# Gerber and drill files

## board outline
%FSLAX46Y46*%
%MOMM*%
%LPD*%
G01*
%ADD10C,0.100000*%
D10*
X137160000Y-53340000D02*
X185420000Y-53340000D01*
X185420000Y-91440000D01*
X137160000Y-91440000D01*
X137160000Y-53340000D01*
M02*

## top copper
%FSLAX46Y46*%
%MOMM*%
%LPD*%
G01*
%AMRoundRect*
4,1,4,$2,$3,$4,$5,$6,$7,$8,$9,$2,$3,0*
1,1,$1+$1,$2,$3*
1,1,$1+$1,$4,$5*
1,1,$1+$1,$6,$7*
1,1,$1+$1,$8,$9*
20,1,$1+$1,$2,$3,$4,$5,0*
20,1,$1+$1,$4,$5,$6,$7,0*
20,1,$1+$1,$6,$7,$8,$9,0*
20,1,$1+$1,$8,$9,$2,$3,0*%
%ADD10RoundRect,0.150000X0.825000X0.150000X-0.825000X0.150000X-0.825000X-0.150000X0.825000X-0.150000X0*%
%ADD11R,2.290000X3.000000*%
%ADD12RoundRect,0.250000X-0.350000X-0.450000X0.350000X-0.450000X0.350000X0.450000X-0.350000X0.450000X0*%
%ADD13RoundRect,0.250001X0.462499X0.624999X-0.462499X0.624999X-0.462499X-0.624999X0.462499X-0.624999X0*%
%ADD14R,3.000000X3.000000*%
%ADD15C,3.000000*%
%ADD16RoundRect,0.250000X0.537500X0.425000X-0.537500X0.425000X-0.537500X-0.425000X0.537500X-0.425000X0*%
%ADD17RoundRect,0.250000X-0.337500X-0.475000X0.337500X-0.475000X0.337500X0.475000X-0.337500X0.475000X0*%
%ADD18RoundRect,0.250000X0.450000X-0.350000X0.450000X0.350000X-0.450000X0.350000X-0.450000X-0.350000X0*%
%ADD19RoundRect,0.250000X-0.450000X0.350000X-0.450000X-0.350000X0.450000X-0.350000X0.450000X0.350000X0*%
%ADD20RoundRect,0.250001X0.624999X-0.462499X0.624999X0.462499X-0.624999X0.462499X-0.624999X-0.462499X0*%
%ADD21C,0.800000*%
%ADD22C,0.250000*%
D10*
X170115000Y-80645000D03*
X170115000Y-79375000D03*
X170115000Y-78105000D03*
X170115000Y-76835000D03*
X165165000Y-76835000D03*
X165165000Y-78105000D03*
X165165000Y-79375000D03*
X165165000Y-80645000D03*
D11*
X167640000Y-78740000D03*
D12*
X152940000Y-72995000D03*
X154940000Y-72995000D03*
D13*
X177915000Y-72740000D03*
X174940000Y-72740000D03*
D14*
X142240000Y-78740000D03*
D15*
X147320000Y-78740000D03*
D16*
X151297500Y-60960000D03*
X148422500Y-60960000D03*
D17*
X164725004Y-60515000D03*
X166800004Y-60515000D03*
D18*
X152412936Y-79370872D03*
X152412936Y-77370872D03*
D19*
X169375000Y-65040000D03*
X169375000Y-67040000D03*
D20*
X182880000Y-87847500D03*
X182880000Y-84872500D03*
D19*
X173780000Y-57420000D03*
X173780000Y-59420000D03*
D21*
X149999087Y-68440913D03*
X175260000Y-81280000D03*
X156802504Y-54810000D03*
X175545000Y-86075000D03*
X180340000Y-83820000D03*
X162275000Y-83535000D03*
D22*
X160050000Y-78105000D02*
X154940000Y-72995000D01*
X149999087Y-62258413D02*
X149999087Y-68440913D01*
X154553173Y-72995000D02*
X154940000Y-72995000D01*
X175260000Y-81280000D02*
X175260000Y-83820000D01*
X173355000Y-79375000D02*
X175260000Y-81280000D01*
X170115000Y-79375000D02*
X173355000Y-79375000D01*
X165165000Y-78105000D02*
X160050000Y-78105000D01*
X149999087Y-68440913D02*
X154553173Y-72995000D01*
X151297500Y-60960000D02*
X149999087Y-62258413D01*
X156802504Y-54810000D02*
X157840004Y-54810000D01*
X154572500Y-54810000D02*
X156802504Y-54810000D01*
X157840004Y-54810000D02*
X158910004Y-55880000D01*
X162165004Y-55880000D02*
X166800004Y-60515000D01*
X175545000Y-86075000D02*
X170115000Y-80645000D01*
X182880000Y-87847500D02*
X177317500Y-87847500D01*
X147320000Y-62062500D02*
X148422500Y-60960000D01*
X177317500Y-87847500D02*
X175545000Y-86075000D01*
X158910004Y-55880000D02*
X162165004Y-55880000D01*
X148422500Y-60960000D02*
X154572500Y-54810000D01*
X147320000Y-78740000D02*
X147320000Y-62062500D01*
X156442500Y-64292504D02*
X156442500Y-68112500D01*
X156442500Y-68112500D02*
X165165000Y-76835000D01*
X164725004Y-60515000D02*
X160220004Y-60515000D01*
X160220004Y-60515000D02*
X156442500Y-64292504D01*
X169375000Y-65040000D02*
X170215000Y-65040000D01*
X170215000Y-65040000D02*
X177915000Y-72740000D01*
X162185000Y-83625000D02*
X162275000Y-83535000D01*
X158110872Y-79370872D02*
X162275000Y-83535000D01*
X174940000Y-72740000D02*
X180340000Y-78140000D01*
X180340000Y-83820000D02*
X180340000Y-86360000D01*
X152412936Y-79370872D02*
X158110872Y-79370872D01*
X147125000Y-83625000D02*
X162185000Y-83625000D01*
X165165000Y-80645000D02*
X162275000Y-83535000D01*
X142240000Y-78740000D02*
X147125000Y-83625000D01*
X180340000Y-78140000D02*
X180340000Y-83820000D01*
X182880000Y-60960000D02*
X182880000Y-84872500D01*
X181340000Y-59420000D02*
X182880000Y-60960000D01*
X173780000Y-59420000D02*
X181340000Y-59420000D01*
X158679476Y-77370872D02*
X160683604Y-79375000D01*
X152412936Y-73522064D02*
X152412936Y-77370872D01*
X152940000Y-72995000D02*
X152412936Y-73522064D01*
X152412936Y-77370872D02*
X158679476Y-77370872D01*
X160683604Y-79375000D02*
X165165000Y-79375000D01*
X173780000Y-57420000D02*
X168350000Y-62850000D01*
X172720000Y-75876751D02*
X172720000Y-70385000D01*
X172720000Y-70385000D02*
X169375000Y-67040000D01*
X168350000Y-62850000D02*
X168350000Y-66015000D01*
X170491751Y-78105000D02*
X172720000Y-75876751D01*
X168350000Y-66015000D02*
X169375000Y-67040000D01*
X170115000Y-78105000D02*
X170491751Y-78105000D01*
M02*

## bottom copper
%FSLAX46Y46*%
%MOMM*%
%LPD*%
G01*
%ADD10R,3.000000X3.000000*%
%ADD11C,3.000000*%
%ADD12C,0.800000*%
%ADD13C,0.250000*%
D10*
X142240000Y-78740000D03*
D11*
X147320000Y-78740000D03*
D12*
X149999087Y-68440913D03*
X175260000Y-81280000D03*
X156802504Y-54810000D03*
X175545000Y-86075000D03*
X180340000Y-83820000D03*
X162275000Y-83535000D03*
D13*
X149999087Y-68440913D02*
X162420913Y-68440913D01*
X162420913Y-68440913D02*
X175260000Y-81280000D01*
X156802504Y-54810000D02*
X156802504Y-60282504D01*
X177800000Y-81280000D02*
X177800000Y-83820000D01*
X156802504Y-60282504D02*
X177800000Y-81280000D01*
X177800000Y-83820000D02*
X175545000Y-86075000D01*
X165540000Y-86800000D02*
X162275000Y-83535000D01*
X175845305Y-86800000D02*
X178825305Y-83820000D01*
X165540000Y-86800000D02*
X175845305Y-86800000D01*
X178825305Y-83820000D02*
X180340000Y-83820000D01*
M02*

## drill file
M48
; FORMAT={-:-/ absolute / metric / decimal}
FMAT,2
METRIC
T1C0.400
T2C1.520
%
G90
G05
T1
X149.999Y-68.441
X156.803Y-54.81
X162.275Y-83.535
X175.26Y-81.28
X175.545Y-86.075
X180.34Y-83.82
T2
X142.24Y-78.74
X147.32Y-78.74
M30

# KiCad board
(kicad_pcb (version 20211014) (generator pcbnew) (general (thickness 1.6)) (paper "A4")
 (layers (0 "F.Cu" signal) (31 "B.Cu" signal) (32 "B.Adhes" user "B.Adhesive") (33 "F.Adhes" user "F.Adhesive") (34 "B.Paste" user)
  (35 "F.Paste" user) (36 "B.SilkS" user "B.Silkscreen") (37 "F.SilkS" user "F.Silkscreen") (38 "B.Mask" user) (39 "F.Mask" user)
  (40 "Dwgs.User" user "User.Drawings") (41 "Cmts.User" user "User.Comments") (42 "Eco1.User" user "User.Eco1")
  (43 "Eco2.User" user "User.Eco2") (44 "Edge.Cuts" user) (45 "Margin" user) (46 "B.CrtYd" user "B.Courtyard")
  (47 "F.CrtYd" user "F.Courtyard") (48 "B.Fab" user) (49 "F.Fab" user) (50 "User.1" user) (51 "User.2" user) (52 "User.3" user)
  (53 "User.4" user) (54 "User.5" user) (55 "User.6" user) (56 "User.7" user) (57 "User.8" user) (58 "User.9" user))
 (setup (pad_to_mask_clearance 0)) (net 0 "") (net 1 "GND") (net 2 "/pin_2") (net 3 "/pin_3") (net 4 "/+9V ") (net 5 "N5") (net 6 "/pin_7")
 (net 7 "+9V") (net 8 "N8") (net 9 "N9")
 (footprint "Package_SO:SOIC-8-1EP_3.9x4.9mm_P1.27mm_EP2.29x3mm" (layer "F.Cu") (at 167.64 78.74 180)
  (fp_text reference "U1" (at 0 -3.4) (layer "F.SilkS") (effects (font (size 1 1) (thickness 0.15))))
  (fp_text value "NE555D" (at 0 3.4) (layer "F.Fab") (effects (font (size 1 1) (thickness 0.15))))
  (pad "" smd roundrect (at 0.57 0.75 180) (size 0.92 1.21) (layers "F.Paste") (roundrect_rratio 0.25))
  (pad "" smd roundrect (at -0.57 0.75 180) (size 0.92 1.21) (layers "F.Paste") (roundrect_rratio 0.25))
  (pad "" smd roundrect (at 0.57 -0.75 180) (size 0.92 1.21) (layers "F.Paste") (roundrect_rratio 0.25))
  (pad "" smd roundrect (at -0.57 -0.75 180) (size 0.92 1.21) (layers "F.Paste") (roundrect_rratio 0.25))
  (pad "1" smd roundrect (at -2.475 -1.905 180) (size 1.95 0.6) (layers "F.Cu" "F.Paste" "F.Mask") (roundrect_rratio 0.25) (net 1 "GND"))
  (pad "2" smd roundrect (at -2.475 -0.635 180) (size 1.95 0.6) (layers "F.Cu" "F.Paste" "F.Mask") (roundrect_rratio 0.25) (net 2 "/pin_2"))
  (pad "3" smd roundrect (at -2.475 0.635 180) (size 1.95 0.6) (layers "F.Cu" "F.Paste" "F.Mask") (roundrect_rratio 0.25) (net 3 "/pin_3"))
  (pad "4" smd roundrect (at -2.475 1.905 180) (size 1.95 0.6) (layers "F.Cu" "F.Paste" "F.Mask") (roundrect_rratio 0.25) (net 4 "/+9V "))
  (pad "5" smd roundrect (at 2.475 1.905 180) (size 1.95 0.6) (layers "F.Cu" "F.Paste" "F.Mask") (roundrect_rratio 0.25) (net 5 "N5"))
  (pad "6" smd roundrect (at 2.475 0.635 180) (size 1.95 0.6) (layers "F.Cu" "F.Paste" "F.Mask") (roundrect_rratio 0.25) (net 2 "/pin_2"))
  (pad "7" smd roundrect (at 2.475 -0.635 180) (size 1.95 0.6) (layers "F.Cu" "F.Paste" "F.Mask") (roundrect_rratio 0.25) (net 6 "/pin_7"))
  (pad "8" smd roundrect (at 2.475 -1.905 180) (size 1.95 0.6) (layers "F.Cu" "F.Paste" "F.Mask") (roundrect_rratio 0.25) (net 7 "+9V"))
  (pad "9" smd rect (at 0 0 180) (size 2.29 3) (layers "F.Cu" "F.Mask")))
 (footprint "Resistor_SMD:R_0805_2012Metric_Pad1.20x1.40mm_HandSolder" (layer "F.Cu") (at 153.94 72.995)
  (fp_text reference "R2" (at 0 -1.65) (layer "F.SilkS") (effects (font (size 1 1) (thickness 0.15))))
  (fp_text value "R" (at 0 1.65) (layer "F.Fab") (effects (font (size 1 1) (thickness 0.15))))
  (pad "1" smd roundrect (at -1 0) (size 1.2 1.4) (layers "F.Cu" "F.Paste" "F.Mask") (roundrect_rratio 0.2083333333) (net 6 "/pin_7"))
  (pad "2" smd roundrect (at 1 0) (size 1.2 1.4) (layers "F.Cu" "F.Paste" "F.Mask") (roundrect_rratio 0.2083333333) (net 2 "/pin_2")))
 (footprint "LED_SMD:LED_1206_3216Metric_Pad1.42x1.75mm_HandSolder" (layer "F.Cu") (at 176.4275 72.74 180)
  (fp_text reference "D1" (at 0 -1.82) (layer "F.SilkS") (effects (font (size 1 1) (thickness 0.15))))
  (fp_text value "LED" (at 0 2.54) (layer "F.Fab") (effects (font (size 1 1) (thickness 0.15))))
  (pad "1" smd roundrect (at -1.4875 0 180) (size 1.425 1.75) (layers "F.Cu" "F.Paste" "F.Mask") (roundrect_rratio 0.1754392982)
   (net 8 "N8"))
  (pad "2" smd roundrect (at 1.4875 0 180) (size 1.425 1.75) (layers "F.Cu" "F.Paste" "F.Mask") (roundrect_rratio 0.1754392982)
   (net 7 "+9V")))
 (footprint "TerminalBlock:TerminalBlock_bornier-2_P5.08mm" (layer "F.Cu") (at 142.24 78.74)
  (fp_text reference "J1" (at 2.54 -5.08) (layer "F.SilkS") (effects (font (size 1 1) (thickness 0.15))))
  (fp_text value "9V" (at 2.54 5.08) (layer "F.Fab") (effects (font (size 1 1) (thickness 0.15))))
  (pad "1" thru_hole rect (at 0 0) (size 3 3) (drill 1.52) (layers *.Cu *.Mask) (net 7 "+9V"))
  (pad "2" thru_hole circle (at 5.08 0) (size 3 3) (drill 1.52) (layers *.Cu *.Mask) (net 1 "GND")))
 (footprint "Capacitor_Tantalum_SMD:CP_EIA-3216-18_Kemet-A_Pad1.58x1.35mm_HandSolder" (layer "F.Cu") (at 149.86 60.96 180)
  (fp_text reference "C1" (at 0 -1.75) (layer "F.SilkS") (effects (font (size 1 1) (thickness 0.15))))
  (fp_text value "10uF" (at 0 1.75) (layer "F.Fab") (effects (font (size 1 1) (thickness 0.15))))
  (pad "1" smd roundrect (at -1.4375 0 180) (size 1.575 1.35) (layers "F.Cu" "F.Paste" "F.Mask") (roundrect_rratio 0.1851851852)
   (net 2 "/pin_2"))
  (pad "2" smd roundrect (at 1.4375 0 180) (size 1.575 1.35) (layers "F.Cu" "F.Paste" "F.Mask") (roundrect_rratio 0.1851851852)
   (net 1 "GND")))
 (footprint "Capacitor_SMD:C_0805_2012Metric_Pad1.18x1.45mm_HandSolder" (layer "F.Cu") (at 165.762504 60.515)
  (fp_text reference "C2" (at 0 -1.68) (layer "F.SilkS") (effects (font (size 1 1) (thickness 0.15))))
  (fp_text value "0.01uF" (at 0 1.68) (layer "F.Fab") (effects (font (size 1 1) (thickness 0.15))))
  (pad "1" smd roundrect (at -1.0375 0) (size 1.175 1.45) (layers "F.Cu" "F.Paste" "F.Mask") (roundrect_rratio 0.2127659574) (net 5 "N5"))
  (pad "2" smd roundrect (at 1.0375 0) (size 1.175 1.45) (layers "F.Cu" "F.Paste" "F.Mask") (roundrect_rratio 0.2127659574) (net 1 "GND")))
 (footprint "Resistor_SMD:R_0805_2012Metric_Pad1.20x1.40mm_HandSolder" (layer "F.Cu") (at 152.412936 78.370872 90)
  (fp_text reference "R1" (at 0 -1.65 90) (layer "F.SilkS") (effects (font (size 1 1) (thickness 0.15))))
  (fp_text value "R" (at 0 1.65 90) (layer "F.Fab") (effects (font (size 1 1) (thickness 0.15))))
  (pad "1" smd roundrect (at -1 0 90) (size 1.2 1.4) (layers "F.Cu" "F.Paste" "F.Mask") (roundrect_rratio 0.2083333333) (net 7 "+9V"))
  (pad "2" smd roundrect (at 1 0 90) (size 1.2 1.4) (layers "F.Cu" "F.Paste" "F.Mask") (roundrect_rratio 0.2083333333) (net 6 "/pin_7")))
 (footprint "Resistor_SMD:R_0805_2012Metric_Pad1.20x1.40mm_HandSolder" (layer "F.Cu") (at 169.375 66.04 -90)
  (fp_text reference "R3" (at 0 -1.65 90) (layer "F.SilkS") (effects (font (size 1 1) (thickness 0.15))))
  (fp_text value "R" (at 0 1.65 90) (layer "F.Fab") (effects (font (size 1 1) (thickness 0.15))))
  (pad "1" smd roundrect (at -1 0 270) (size 1.2 1.4) (layers "F.Cu" "F.Paste" "F.Mask") (roundrect_rratio 0.2083333333) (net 8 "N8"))
  (pad "2" smd roundrect (at 1 0 270) (size 1.2 1.4) (layers "F.Cu" "F.Paste" "F.Mask") (roundrect_rratio 0.2083333333) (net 3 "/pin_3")))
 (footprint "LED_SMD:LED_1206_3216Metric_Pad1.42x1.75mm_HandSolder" (layer "F.Cu") (at 182.88 86.36 90)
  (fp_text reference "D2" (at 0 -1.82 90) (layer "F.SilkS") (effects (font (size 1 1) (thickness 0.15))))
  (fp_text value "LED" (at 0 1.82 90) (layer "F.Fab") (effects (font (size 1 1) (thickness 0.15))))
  (pad "1" smd roundrect (at -1.4875 0 90) (size 1.425 1.75) (layers "F.Cu" "F.Paste" "F.Mask") (roundrect_rratio 0.1754392982)
   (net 1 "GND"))
  (pad "2" smd roundrect (at 1.4875 0 90) (size 1.425 1.75) (layers "F.Cu" "F.Paste" "F.Mask") (roundrect_rratio 0.1754392982) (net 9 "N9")))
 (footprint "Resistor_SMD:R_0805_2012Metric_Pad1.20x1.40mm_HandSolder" (layer "F.Cu") (at 173.78 58.42 -90)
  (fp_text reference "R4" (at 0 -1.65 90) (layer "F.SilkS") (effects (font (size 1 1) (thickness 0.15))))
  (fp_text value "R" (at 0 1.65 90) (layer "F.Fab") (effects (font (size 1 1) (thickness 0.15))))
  (pad "1" smd roundrect (at -1 0 270) (size 1.2 1.4) (layers "F.Cu" "F.Paste" "F.Mask") (roundrect_rratio 0.2083333333) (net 3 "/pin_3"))
  (pad "2" smd roundrect (at 1 0 270) (size 1.2 1.4) (layers "F.Cu" "F.Paste" "F.Mask") (roundrect_rratio 0.2083333333) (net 9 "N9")))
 (gr_rect (start 185.42 91.44) (end 137.16 53.34) (layer "Edge.Cuts") (width 0.1) (fill none))
 (segment (start 160.05 78.105) (end 154.94 72.995) (width 0.25) (layer "F.Cu") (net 2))
 (segment (start 149.999087 62.258413) (end 149.999087 68.440913) (width 0.25) (layer "F.Cu") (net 2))
 (segment (start 154.553173 72.995) (end 154.94 72.995) (width 0.25) (layer "F.Cu") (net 2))
 (segment (start 175.26 81.28) (end 175.26 83.82) (width 0.25) (layer "F.Cu") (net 2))
 (segment (start 173.355 79.375) (end 175.26 81.28) (width 0.25) (layer "F.Cu") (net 2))
 (segment (start 170.115 79.375) (end 173.355 79.375) (width 0.25) (layer "F.Cu") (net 2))
 (segment (start 165.165 78.105) (end 160.05 78.105) (width 0.25) (layer "F.Cu") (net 2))
 (segment (start 149.999087 68.440913) (end 154.553173 72.995) (width 0.25) (layer "F.Cu") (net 2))
 (segment (start 151.2975 60.96) (end 149.999087 62.258413) (width 0.25) (layer "F.Cu") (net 2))
 (via (at 149.999087 68.440913) (size 0.8) (drill 0.4) (layers "F.Cu" "B.Cu") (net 2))
 (via (at 175.26 81.28) (size 0.8) (drill 0.4) (layers "F.Cu" "B.Cu") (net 2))
 (segment (start 149.999087 68.440913) (end 162.420913 68.440913) (width 0.25) (layer "B.Cu") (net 2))
 (segment (start 162.420913 68.440913) (end 175.26 81.28) (width 0.25) (layer "B.Cu") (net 2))
 (segment (start 156.802504 54.81) (end 157.840004 54.81) (width 0.25) (layer "F.Cu") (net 1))
 (segment (start 154.5725 54.81) (end 156.802504 54.81) (width 0.25) (layer "F.Cu") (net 1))
 (segment (start 157.840004 54.81) (end 158.910004 55.88) (width 0.25) (layer "F.Cu") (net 1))
 (segment (start 162.165004 55.88) (end 166.800004 60.515) (width 0.25) (layer "F.Cu") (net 1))
 (segment (start 175.545 86.075) (end 170.115 80.645) (width 0.25) (layer "F.Cu") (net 1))
 (segment (start 182.88 87.8475) (end 177.3175 87.8475) (width 0.25) (layer "F.Cu") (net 1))
 (segment (start 147.32 62.0625) (end 148.4225 60.96) (width 0.25) (layer "F.Cu") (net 1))
 (segment (start 177.3175 87.8475) (end 175.545 86.075) (width 0.25) (layer "F.Cu") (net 1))
 (segment (start 158.910004 55.88) (end 162.165004 55.88) (width 0.25) (layer "F.Cu") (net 1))
 (segment (start 148.4225 60.96) (end 154.5725 54.81) (width 0.25) (layer "F.Cu") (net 1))
 (segment (start 147.32 78.74) (end 147.32 62.0625) (width 0.25) (layer "F.Cu") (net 1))
 (via (at 156.802504 54.81) (size 0.8) (drill 0.4) (layers "F.Cu" "B.Cu") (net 1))
 (via (at 175.545 86.075) (size 0.8) (drill 0.4) (layers "F.Cu" "B.Cu") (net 1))
 (segment (start 156.802504 54.81) (end 156.802504 60.282504) (width 0.25) (layer "B.Cu") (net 1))
 (segment (start 177.8 81.28) (end 177.8 83.82) (width 0.25) (layer "B.Cu") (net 1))
 (segment (start 156.802504 60.282504) (end 177.8 81.28) (width 0.25) (layer "B.Cu") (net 1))
 (segment (start 177.8 83.82) (end 175.545 86.075) (width 0.25) (layer "B.Cu") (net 1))
 (segment (start 156.4425 64.292504) (end 156.4425 68.1125) (width 0.25) (layer "F.Cu") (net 5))
 (segment (start 156.4425 68.1125) (end 165.165 76.835) (width 0.25) (layer "F.Cu") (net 5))
 (segment (start 164.725004 60.515) (end 160.220004 60.515) (width 0.25) (layer "F.Cu") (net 5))
 (segment (start 160.220004 60.515) (end 156.4425 64.292504) (width 0.25) (layer "F.Cu") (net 5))
 (segment (start 169.375 65.04) (end 170.215 65.04) (width 0.25) (layer "F.Cu") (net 8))
 (segment (start 170.215 65.04) (end 177.915 72.74) (width 0.25) (layer "F.Cu") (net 8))
 (segment (start 162.185 83.625) (end 162.275 83.535) (width 0.25) (layer "F.Cu") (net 7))
 (segment (start 158.110872 79.370872) (end 162.275 83.535) (width 0.25) (layer "F.Cu") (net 7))
 (segment (start 174.94 72.74) (end 180.34 78.14) (width 0.25) (layer "F.Cu") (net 7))
 (segment (start 180.34 83.82) (end 180.34 86.36) (width 0.25) (layer "F.Cu") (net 7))
 (segment (start 152.412936 79.370872) (end 158.110872 79.370872) (width 0.25) (layer "F.Cu") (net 7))
 (segment (start 147.125 83.625) (end 162.185 83.625) (width 0.25) (layer "F.Cu") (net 7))
 (segment (start 165.165 80.645) (end 162.275 83.535) (width 0.25) (layer "F.Cu") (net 7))
 (segment (start 142.24 78.74) (end 147.125 83.625) (width 0.25) (layer "F.Cu") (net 7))
 (segment (start 180.34 78.14) (end 180.34 83.82) (width 0.25) (layer "F.Cu") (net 7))
 (via (at 180.34 83.82) (size 0.8) (drill 0.4) (layers "F.Cu" "B.Cu") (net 7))
 (via (at 162.275 83.535) (size 0.8) (drill 0.4) (layers "F.Cu" "B.Cu") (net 7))
 (segment (start 165.54 86.8) (end 162.275 83.535) (width 0.25) (layer "B.Cu") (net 7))
 (segment (start 175.845305 86.8) (end 178.825305 83.82) (width 0.25) (layer "B.Cu") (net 7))
 (segment (start 165.54 86.8) (end 175.845305 86.8) (width 0.25) (layer "B.Cu") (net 7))
 (segment (start 178.825305 83.82) (end 180.34 83.82) (width 0.25) (layer "B.Cu") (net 7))
 (segment (start 182.88 60.96) (end 182.88 84.8725) (width 0.25) (layer "F.Cu") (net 9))
 (segment (start 181.34 59.42) (end 182.88 60.96) (width 0.25) (layer "F.Cu") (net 9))
 (segment (start 173.78 59.42) (end 181.34 59.42) (width 0.25) (layer "F.Cu") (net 9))
 (segment (start 158.679476 77.370872) (end 160.683604 79.375) (width 0.25) (layer "F.Cu") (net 6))
 (segment (start 152.412936 73.522064) (end 152.412936 77.370872) (width 0.25) (layer "F.Cu") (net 6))
 (segment (start 152.94 72.995) (end 152.412936 73.522064) (width 0.25) (layer "F.Cu") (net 6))
 (segment (start 152.412936 77.370872) (end 158.679476 77.370872) (width 0.25) (layer "F.Cu") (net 6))
 (segment (start 160.683604 79.375) (end 165.165 79.375) (width 0.25) (layer "F.Cu") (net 6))
 (segment (start 173.78 57.42) (end 168.35 62.85) (width 0.25) (layer "F.Cu") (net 3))
 (segment (start 172.72 75.876751) (end 172.72 70.385) (width 0.25) (layer "F.Cu") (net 3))
 (segment (start 172.72 70.385) (end 169.375 67.04) (width 0.25) (layer "F.Cu") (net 3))
 (segment (start 168.35 62.85) (end 168.35 66.015) (width 0.25) (layer "F.Cu") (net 3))
 (segment (start 170.491751 78.105) (end 172.72 75.876751) (width 0.25) (layer "F.Cu") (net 3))
 (segment (start 168.35 66.015) (end 169.375 67.04) (width 0.25) (layer "F.Cu") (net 3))
 (segment (start 170.115 78.105) (end 170.491751 78.105) (width 0.25) (layer "F.Cu") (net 3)))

